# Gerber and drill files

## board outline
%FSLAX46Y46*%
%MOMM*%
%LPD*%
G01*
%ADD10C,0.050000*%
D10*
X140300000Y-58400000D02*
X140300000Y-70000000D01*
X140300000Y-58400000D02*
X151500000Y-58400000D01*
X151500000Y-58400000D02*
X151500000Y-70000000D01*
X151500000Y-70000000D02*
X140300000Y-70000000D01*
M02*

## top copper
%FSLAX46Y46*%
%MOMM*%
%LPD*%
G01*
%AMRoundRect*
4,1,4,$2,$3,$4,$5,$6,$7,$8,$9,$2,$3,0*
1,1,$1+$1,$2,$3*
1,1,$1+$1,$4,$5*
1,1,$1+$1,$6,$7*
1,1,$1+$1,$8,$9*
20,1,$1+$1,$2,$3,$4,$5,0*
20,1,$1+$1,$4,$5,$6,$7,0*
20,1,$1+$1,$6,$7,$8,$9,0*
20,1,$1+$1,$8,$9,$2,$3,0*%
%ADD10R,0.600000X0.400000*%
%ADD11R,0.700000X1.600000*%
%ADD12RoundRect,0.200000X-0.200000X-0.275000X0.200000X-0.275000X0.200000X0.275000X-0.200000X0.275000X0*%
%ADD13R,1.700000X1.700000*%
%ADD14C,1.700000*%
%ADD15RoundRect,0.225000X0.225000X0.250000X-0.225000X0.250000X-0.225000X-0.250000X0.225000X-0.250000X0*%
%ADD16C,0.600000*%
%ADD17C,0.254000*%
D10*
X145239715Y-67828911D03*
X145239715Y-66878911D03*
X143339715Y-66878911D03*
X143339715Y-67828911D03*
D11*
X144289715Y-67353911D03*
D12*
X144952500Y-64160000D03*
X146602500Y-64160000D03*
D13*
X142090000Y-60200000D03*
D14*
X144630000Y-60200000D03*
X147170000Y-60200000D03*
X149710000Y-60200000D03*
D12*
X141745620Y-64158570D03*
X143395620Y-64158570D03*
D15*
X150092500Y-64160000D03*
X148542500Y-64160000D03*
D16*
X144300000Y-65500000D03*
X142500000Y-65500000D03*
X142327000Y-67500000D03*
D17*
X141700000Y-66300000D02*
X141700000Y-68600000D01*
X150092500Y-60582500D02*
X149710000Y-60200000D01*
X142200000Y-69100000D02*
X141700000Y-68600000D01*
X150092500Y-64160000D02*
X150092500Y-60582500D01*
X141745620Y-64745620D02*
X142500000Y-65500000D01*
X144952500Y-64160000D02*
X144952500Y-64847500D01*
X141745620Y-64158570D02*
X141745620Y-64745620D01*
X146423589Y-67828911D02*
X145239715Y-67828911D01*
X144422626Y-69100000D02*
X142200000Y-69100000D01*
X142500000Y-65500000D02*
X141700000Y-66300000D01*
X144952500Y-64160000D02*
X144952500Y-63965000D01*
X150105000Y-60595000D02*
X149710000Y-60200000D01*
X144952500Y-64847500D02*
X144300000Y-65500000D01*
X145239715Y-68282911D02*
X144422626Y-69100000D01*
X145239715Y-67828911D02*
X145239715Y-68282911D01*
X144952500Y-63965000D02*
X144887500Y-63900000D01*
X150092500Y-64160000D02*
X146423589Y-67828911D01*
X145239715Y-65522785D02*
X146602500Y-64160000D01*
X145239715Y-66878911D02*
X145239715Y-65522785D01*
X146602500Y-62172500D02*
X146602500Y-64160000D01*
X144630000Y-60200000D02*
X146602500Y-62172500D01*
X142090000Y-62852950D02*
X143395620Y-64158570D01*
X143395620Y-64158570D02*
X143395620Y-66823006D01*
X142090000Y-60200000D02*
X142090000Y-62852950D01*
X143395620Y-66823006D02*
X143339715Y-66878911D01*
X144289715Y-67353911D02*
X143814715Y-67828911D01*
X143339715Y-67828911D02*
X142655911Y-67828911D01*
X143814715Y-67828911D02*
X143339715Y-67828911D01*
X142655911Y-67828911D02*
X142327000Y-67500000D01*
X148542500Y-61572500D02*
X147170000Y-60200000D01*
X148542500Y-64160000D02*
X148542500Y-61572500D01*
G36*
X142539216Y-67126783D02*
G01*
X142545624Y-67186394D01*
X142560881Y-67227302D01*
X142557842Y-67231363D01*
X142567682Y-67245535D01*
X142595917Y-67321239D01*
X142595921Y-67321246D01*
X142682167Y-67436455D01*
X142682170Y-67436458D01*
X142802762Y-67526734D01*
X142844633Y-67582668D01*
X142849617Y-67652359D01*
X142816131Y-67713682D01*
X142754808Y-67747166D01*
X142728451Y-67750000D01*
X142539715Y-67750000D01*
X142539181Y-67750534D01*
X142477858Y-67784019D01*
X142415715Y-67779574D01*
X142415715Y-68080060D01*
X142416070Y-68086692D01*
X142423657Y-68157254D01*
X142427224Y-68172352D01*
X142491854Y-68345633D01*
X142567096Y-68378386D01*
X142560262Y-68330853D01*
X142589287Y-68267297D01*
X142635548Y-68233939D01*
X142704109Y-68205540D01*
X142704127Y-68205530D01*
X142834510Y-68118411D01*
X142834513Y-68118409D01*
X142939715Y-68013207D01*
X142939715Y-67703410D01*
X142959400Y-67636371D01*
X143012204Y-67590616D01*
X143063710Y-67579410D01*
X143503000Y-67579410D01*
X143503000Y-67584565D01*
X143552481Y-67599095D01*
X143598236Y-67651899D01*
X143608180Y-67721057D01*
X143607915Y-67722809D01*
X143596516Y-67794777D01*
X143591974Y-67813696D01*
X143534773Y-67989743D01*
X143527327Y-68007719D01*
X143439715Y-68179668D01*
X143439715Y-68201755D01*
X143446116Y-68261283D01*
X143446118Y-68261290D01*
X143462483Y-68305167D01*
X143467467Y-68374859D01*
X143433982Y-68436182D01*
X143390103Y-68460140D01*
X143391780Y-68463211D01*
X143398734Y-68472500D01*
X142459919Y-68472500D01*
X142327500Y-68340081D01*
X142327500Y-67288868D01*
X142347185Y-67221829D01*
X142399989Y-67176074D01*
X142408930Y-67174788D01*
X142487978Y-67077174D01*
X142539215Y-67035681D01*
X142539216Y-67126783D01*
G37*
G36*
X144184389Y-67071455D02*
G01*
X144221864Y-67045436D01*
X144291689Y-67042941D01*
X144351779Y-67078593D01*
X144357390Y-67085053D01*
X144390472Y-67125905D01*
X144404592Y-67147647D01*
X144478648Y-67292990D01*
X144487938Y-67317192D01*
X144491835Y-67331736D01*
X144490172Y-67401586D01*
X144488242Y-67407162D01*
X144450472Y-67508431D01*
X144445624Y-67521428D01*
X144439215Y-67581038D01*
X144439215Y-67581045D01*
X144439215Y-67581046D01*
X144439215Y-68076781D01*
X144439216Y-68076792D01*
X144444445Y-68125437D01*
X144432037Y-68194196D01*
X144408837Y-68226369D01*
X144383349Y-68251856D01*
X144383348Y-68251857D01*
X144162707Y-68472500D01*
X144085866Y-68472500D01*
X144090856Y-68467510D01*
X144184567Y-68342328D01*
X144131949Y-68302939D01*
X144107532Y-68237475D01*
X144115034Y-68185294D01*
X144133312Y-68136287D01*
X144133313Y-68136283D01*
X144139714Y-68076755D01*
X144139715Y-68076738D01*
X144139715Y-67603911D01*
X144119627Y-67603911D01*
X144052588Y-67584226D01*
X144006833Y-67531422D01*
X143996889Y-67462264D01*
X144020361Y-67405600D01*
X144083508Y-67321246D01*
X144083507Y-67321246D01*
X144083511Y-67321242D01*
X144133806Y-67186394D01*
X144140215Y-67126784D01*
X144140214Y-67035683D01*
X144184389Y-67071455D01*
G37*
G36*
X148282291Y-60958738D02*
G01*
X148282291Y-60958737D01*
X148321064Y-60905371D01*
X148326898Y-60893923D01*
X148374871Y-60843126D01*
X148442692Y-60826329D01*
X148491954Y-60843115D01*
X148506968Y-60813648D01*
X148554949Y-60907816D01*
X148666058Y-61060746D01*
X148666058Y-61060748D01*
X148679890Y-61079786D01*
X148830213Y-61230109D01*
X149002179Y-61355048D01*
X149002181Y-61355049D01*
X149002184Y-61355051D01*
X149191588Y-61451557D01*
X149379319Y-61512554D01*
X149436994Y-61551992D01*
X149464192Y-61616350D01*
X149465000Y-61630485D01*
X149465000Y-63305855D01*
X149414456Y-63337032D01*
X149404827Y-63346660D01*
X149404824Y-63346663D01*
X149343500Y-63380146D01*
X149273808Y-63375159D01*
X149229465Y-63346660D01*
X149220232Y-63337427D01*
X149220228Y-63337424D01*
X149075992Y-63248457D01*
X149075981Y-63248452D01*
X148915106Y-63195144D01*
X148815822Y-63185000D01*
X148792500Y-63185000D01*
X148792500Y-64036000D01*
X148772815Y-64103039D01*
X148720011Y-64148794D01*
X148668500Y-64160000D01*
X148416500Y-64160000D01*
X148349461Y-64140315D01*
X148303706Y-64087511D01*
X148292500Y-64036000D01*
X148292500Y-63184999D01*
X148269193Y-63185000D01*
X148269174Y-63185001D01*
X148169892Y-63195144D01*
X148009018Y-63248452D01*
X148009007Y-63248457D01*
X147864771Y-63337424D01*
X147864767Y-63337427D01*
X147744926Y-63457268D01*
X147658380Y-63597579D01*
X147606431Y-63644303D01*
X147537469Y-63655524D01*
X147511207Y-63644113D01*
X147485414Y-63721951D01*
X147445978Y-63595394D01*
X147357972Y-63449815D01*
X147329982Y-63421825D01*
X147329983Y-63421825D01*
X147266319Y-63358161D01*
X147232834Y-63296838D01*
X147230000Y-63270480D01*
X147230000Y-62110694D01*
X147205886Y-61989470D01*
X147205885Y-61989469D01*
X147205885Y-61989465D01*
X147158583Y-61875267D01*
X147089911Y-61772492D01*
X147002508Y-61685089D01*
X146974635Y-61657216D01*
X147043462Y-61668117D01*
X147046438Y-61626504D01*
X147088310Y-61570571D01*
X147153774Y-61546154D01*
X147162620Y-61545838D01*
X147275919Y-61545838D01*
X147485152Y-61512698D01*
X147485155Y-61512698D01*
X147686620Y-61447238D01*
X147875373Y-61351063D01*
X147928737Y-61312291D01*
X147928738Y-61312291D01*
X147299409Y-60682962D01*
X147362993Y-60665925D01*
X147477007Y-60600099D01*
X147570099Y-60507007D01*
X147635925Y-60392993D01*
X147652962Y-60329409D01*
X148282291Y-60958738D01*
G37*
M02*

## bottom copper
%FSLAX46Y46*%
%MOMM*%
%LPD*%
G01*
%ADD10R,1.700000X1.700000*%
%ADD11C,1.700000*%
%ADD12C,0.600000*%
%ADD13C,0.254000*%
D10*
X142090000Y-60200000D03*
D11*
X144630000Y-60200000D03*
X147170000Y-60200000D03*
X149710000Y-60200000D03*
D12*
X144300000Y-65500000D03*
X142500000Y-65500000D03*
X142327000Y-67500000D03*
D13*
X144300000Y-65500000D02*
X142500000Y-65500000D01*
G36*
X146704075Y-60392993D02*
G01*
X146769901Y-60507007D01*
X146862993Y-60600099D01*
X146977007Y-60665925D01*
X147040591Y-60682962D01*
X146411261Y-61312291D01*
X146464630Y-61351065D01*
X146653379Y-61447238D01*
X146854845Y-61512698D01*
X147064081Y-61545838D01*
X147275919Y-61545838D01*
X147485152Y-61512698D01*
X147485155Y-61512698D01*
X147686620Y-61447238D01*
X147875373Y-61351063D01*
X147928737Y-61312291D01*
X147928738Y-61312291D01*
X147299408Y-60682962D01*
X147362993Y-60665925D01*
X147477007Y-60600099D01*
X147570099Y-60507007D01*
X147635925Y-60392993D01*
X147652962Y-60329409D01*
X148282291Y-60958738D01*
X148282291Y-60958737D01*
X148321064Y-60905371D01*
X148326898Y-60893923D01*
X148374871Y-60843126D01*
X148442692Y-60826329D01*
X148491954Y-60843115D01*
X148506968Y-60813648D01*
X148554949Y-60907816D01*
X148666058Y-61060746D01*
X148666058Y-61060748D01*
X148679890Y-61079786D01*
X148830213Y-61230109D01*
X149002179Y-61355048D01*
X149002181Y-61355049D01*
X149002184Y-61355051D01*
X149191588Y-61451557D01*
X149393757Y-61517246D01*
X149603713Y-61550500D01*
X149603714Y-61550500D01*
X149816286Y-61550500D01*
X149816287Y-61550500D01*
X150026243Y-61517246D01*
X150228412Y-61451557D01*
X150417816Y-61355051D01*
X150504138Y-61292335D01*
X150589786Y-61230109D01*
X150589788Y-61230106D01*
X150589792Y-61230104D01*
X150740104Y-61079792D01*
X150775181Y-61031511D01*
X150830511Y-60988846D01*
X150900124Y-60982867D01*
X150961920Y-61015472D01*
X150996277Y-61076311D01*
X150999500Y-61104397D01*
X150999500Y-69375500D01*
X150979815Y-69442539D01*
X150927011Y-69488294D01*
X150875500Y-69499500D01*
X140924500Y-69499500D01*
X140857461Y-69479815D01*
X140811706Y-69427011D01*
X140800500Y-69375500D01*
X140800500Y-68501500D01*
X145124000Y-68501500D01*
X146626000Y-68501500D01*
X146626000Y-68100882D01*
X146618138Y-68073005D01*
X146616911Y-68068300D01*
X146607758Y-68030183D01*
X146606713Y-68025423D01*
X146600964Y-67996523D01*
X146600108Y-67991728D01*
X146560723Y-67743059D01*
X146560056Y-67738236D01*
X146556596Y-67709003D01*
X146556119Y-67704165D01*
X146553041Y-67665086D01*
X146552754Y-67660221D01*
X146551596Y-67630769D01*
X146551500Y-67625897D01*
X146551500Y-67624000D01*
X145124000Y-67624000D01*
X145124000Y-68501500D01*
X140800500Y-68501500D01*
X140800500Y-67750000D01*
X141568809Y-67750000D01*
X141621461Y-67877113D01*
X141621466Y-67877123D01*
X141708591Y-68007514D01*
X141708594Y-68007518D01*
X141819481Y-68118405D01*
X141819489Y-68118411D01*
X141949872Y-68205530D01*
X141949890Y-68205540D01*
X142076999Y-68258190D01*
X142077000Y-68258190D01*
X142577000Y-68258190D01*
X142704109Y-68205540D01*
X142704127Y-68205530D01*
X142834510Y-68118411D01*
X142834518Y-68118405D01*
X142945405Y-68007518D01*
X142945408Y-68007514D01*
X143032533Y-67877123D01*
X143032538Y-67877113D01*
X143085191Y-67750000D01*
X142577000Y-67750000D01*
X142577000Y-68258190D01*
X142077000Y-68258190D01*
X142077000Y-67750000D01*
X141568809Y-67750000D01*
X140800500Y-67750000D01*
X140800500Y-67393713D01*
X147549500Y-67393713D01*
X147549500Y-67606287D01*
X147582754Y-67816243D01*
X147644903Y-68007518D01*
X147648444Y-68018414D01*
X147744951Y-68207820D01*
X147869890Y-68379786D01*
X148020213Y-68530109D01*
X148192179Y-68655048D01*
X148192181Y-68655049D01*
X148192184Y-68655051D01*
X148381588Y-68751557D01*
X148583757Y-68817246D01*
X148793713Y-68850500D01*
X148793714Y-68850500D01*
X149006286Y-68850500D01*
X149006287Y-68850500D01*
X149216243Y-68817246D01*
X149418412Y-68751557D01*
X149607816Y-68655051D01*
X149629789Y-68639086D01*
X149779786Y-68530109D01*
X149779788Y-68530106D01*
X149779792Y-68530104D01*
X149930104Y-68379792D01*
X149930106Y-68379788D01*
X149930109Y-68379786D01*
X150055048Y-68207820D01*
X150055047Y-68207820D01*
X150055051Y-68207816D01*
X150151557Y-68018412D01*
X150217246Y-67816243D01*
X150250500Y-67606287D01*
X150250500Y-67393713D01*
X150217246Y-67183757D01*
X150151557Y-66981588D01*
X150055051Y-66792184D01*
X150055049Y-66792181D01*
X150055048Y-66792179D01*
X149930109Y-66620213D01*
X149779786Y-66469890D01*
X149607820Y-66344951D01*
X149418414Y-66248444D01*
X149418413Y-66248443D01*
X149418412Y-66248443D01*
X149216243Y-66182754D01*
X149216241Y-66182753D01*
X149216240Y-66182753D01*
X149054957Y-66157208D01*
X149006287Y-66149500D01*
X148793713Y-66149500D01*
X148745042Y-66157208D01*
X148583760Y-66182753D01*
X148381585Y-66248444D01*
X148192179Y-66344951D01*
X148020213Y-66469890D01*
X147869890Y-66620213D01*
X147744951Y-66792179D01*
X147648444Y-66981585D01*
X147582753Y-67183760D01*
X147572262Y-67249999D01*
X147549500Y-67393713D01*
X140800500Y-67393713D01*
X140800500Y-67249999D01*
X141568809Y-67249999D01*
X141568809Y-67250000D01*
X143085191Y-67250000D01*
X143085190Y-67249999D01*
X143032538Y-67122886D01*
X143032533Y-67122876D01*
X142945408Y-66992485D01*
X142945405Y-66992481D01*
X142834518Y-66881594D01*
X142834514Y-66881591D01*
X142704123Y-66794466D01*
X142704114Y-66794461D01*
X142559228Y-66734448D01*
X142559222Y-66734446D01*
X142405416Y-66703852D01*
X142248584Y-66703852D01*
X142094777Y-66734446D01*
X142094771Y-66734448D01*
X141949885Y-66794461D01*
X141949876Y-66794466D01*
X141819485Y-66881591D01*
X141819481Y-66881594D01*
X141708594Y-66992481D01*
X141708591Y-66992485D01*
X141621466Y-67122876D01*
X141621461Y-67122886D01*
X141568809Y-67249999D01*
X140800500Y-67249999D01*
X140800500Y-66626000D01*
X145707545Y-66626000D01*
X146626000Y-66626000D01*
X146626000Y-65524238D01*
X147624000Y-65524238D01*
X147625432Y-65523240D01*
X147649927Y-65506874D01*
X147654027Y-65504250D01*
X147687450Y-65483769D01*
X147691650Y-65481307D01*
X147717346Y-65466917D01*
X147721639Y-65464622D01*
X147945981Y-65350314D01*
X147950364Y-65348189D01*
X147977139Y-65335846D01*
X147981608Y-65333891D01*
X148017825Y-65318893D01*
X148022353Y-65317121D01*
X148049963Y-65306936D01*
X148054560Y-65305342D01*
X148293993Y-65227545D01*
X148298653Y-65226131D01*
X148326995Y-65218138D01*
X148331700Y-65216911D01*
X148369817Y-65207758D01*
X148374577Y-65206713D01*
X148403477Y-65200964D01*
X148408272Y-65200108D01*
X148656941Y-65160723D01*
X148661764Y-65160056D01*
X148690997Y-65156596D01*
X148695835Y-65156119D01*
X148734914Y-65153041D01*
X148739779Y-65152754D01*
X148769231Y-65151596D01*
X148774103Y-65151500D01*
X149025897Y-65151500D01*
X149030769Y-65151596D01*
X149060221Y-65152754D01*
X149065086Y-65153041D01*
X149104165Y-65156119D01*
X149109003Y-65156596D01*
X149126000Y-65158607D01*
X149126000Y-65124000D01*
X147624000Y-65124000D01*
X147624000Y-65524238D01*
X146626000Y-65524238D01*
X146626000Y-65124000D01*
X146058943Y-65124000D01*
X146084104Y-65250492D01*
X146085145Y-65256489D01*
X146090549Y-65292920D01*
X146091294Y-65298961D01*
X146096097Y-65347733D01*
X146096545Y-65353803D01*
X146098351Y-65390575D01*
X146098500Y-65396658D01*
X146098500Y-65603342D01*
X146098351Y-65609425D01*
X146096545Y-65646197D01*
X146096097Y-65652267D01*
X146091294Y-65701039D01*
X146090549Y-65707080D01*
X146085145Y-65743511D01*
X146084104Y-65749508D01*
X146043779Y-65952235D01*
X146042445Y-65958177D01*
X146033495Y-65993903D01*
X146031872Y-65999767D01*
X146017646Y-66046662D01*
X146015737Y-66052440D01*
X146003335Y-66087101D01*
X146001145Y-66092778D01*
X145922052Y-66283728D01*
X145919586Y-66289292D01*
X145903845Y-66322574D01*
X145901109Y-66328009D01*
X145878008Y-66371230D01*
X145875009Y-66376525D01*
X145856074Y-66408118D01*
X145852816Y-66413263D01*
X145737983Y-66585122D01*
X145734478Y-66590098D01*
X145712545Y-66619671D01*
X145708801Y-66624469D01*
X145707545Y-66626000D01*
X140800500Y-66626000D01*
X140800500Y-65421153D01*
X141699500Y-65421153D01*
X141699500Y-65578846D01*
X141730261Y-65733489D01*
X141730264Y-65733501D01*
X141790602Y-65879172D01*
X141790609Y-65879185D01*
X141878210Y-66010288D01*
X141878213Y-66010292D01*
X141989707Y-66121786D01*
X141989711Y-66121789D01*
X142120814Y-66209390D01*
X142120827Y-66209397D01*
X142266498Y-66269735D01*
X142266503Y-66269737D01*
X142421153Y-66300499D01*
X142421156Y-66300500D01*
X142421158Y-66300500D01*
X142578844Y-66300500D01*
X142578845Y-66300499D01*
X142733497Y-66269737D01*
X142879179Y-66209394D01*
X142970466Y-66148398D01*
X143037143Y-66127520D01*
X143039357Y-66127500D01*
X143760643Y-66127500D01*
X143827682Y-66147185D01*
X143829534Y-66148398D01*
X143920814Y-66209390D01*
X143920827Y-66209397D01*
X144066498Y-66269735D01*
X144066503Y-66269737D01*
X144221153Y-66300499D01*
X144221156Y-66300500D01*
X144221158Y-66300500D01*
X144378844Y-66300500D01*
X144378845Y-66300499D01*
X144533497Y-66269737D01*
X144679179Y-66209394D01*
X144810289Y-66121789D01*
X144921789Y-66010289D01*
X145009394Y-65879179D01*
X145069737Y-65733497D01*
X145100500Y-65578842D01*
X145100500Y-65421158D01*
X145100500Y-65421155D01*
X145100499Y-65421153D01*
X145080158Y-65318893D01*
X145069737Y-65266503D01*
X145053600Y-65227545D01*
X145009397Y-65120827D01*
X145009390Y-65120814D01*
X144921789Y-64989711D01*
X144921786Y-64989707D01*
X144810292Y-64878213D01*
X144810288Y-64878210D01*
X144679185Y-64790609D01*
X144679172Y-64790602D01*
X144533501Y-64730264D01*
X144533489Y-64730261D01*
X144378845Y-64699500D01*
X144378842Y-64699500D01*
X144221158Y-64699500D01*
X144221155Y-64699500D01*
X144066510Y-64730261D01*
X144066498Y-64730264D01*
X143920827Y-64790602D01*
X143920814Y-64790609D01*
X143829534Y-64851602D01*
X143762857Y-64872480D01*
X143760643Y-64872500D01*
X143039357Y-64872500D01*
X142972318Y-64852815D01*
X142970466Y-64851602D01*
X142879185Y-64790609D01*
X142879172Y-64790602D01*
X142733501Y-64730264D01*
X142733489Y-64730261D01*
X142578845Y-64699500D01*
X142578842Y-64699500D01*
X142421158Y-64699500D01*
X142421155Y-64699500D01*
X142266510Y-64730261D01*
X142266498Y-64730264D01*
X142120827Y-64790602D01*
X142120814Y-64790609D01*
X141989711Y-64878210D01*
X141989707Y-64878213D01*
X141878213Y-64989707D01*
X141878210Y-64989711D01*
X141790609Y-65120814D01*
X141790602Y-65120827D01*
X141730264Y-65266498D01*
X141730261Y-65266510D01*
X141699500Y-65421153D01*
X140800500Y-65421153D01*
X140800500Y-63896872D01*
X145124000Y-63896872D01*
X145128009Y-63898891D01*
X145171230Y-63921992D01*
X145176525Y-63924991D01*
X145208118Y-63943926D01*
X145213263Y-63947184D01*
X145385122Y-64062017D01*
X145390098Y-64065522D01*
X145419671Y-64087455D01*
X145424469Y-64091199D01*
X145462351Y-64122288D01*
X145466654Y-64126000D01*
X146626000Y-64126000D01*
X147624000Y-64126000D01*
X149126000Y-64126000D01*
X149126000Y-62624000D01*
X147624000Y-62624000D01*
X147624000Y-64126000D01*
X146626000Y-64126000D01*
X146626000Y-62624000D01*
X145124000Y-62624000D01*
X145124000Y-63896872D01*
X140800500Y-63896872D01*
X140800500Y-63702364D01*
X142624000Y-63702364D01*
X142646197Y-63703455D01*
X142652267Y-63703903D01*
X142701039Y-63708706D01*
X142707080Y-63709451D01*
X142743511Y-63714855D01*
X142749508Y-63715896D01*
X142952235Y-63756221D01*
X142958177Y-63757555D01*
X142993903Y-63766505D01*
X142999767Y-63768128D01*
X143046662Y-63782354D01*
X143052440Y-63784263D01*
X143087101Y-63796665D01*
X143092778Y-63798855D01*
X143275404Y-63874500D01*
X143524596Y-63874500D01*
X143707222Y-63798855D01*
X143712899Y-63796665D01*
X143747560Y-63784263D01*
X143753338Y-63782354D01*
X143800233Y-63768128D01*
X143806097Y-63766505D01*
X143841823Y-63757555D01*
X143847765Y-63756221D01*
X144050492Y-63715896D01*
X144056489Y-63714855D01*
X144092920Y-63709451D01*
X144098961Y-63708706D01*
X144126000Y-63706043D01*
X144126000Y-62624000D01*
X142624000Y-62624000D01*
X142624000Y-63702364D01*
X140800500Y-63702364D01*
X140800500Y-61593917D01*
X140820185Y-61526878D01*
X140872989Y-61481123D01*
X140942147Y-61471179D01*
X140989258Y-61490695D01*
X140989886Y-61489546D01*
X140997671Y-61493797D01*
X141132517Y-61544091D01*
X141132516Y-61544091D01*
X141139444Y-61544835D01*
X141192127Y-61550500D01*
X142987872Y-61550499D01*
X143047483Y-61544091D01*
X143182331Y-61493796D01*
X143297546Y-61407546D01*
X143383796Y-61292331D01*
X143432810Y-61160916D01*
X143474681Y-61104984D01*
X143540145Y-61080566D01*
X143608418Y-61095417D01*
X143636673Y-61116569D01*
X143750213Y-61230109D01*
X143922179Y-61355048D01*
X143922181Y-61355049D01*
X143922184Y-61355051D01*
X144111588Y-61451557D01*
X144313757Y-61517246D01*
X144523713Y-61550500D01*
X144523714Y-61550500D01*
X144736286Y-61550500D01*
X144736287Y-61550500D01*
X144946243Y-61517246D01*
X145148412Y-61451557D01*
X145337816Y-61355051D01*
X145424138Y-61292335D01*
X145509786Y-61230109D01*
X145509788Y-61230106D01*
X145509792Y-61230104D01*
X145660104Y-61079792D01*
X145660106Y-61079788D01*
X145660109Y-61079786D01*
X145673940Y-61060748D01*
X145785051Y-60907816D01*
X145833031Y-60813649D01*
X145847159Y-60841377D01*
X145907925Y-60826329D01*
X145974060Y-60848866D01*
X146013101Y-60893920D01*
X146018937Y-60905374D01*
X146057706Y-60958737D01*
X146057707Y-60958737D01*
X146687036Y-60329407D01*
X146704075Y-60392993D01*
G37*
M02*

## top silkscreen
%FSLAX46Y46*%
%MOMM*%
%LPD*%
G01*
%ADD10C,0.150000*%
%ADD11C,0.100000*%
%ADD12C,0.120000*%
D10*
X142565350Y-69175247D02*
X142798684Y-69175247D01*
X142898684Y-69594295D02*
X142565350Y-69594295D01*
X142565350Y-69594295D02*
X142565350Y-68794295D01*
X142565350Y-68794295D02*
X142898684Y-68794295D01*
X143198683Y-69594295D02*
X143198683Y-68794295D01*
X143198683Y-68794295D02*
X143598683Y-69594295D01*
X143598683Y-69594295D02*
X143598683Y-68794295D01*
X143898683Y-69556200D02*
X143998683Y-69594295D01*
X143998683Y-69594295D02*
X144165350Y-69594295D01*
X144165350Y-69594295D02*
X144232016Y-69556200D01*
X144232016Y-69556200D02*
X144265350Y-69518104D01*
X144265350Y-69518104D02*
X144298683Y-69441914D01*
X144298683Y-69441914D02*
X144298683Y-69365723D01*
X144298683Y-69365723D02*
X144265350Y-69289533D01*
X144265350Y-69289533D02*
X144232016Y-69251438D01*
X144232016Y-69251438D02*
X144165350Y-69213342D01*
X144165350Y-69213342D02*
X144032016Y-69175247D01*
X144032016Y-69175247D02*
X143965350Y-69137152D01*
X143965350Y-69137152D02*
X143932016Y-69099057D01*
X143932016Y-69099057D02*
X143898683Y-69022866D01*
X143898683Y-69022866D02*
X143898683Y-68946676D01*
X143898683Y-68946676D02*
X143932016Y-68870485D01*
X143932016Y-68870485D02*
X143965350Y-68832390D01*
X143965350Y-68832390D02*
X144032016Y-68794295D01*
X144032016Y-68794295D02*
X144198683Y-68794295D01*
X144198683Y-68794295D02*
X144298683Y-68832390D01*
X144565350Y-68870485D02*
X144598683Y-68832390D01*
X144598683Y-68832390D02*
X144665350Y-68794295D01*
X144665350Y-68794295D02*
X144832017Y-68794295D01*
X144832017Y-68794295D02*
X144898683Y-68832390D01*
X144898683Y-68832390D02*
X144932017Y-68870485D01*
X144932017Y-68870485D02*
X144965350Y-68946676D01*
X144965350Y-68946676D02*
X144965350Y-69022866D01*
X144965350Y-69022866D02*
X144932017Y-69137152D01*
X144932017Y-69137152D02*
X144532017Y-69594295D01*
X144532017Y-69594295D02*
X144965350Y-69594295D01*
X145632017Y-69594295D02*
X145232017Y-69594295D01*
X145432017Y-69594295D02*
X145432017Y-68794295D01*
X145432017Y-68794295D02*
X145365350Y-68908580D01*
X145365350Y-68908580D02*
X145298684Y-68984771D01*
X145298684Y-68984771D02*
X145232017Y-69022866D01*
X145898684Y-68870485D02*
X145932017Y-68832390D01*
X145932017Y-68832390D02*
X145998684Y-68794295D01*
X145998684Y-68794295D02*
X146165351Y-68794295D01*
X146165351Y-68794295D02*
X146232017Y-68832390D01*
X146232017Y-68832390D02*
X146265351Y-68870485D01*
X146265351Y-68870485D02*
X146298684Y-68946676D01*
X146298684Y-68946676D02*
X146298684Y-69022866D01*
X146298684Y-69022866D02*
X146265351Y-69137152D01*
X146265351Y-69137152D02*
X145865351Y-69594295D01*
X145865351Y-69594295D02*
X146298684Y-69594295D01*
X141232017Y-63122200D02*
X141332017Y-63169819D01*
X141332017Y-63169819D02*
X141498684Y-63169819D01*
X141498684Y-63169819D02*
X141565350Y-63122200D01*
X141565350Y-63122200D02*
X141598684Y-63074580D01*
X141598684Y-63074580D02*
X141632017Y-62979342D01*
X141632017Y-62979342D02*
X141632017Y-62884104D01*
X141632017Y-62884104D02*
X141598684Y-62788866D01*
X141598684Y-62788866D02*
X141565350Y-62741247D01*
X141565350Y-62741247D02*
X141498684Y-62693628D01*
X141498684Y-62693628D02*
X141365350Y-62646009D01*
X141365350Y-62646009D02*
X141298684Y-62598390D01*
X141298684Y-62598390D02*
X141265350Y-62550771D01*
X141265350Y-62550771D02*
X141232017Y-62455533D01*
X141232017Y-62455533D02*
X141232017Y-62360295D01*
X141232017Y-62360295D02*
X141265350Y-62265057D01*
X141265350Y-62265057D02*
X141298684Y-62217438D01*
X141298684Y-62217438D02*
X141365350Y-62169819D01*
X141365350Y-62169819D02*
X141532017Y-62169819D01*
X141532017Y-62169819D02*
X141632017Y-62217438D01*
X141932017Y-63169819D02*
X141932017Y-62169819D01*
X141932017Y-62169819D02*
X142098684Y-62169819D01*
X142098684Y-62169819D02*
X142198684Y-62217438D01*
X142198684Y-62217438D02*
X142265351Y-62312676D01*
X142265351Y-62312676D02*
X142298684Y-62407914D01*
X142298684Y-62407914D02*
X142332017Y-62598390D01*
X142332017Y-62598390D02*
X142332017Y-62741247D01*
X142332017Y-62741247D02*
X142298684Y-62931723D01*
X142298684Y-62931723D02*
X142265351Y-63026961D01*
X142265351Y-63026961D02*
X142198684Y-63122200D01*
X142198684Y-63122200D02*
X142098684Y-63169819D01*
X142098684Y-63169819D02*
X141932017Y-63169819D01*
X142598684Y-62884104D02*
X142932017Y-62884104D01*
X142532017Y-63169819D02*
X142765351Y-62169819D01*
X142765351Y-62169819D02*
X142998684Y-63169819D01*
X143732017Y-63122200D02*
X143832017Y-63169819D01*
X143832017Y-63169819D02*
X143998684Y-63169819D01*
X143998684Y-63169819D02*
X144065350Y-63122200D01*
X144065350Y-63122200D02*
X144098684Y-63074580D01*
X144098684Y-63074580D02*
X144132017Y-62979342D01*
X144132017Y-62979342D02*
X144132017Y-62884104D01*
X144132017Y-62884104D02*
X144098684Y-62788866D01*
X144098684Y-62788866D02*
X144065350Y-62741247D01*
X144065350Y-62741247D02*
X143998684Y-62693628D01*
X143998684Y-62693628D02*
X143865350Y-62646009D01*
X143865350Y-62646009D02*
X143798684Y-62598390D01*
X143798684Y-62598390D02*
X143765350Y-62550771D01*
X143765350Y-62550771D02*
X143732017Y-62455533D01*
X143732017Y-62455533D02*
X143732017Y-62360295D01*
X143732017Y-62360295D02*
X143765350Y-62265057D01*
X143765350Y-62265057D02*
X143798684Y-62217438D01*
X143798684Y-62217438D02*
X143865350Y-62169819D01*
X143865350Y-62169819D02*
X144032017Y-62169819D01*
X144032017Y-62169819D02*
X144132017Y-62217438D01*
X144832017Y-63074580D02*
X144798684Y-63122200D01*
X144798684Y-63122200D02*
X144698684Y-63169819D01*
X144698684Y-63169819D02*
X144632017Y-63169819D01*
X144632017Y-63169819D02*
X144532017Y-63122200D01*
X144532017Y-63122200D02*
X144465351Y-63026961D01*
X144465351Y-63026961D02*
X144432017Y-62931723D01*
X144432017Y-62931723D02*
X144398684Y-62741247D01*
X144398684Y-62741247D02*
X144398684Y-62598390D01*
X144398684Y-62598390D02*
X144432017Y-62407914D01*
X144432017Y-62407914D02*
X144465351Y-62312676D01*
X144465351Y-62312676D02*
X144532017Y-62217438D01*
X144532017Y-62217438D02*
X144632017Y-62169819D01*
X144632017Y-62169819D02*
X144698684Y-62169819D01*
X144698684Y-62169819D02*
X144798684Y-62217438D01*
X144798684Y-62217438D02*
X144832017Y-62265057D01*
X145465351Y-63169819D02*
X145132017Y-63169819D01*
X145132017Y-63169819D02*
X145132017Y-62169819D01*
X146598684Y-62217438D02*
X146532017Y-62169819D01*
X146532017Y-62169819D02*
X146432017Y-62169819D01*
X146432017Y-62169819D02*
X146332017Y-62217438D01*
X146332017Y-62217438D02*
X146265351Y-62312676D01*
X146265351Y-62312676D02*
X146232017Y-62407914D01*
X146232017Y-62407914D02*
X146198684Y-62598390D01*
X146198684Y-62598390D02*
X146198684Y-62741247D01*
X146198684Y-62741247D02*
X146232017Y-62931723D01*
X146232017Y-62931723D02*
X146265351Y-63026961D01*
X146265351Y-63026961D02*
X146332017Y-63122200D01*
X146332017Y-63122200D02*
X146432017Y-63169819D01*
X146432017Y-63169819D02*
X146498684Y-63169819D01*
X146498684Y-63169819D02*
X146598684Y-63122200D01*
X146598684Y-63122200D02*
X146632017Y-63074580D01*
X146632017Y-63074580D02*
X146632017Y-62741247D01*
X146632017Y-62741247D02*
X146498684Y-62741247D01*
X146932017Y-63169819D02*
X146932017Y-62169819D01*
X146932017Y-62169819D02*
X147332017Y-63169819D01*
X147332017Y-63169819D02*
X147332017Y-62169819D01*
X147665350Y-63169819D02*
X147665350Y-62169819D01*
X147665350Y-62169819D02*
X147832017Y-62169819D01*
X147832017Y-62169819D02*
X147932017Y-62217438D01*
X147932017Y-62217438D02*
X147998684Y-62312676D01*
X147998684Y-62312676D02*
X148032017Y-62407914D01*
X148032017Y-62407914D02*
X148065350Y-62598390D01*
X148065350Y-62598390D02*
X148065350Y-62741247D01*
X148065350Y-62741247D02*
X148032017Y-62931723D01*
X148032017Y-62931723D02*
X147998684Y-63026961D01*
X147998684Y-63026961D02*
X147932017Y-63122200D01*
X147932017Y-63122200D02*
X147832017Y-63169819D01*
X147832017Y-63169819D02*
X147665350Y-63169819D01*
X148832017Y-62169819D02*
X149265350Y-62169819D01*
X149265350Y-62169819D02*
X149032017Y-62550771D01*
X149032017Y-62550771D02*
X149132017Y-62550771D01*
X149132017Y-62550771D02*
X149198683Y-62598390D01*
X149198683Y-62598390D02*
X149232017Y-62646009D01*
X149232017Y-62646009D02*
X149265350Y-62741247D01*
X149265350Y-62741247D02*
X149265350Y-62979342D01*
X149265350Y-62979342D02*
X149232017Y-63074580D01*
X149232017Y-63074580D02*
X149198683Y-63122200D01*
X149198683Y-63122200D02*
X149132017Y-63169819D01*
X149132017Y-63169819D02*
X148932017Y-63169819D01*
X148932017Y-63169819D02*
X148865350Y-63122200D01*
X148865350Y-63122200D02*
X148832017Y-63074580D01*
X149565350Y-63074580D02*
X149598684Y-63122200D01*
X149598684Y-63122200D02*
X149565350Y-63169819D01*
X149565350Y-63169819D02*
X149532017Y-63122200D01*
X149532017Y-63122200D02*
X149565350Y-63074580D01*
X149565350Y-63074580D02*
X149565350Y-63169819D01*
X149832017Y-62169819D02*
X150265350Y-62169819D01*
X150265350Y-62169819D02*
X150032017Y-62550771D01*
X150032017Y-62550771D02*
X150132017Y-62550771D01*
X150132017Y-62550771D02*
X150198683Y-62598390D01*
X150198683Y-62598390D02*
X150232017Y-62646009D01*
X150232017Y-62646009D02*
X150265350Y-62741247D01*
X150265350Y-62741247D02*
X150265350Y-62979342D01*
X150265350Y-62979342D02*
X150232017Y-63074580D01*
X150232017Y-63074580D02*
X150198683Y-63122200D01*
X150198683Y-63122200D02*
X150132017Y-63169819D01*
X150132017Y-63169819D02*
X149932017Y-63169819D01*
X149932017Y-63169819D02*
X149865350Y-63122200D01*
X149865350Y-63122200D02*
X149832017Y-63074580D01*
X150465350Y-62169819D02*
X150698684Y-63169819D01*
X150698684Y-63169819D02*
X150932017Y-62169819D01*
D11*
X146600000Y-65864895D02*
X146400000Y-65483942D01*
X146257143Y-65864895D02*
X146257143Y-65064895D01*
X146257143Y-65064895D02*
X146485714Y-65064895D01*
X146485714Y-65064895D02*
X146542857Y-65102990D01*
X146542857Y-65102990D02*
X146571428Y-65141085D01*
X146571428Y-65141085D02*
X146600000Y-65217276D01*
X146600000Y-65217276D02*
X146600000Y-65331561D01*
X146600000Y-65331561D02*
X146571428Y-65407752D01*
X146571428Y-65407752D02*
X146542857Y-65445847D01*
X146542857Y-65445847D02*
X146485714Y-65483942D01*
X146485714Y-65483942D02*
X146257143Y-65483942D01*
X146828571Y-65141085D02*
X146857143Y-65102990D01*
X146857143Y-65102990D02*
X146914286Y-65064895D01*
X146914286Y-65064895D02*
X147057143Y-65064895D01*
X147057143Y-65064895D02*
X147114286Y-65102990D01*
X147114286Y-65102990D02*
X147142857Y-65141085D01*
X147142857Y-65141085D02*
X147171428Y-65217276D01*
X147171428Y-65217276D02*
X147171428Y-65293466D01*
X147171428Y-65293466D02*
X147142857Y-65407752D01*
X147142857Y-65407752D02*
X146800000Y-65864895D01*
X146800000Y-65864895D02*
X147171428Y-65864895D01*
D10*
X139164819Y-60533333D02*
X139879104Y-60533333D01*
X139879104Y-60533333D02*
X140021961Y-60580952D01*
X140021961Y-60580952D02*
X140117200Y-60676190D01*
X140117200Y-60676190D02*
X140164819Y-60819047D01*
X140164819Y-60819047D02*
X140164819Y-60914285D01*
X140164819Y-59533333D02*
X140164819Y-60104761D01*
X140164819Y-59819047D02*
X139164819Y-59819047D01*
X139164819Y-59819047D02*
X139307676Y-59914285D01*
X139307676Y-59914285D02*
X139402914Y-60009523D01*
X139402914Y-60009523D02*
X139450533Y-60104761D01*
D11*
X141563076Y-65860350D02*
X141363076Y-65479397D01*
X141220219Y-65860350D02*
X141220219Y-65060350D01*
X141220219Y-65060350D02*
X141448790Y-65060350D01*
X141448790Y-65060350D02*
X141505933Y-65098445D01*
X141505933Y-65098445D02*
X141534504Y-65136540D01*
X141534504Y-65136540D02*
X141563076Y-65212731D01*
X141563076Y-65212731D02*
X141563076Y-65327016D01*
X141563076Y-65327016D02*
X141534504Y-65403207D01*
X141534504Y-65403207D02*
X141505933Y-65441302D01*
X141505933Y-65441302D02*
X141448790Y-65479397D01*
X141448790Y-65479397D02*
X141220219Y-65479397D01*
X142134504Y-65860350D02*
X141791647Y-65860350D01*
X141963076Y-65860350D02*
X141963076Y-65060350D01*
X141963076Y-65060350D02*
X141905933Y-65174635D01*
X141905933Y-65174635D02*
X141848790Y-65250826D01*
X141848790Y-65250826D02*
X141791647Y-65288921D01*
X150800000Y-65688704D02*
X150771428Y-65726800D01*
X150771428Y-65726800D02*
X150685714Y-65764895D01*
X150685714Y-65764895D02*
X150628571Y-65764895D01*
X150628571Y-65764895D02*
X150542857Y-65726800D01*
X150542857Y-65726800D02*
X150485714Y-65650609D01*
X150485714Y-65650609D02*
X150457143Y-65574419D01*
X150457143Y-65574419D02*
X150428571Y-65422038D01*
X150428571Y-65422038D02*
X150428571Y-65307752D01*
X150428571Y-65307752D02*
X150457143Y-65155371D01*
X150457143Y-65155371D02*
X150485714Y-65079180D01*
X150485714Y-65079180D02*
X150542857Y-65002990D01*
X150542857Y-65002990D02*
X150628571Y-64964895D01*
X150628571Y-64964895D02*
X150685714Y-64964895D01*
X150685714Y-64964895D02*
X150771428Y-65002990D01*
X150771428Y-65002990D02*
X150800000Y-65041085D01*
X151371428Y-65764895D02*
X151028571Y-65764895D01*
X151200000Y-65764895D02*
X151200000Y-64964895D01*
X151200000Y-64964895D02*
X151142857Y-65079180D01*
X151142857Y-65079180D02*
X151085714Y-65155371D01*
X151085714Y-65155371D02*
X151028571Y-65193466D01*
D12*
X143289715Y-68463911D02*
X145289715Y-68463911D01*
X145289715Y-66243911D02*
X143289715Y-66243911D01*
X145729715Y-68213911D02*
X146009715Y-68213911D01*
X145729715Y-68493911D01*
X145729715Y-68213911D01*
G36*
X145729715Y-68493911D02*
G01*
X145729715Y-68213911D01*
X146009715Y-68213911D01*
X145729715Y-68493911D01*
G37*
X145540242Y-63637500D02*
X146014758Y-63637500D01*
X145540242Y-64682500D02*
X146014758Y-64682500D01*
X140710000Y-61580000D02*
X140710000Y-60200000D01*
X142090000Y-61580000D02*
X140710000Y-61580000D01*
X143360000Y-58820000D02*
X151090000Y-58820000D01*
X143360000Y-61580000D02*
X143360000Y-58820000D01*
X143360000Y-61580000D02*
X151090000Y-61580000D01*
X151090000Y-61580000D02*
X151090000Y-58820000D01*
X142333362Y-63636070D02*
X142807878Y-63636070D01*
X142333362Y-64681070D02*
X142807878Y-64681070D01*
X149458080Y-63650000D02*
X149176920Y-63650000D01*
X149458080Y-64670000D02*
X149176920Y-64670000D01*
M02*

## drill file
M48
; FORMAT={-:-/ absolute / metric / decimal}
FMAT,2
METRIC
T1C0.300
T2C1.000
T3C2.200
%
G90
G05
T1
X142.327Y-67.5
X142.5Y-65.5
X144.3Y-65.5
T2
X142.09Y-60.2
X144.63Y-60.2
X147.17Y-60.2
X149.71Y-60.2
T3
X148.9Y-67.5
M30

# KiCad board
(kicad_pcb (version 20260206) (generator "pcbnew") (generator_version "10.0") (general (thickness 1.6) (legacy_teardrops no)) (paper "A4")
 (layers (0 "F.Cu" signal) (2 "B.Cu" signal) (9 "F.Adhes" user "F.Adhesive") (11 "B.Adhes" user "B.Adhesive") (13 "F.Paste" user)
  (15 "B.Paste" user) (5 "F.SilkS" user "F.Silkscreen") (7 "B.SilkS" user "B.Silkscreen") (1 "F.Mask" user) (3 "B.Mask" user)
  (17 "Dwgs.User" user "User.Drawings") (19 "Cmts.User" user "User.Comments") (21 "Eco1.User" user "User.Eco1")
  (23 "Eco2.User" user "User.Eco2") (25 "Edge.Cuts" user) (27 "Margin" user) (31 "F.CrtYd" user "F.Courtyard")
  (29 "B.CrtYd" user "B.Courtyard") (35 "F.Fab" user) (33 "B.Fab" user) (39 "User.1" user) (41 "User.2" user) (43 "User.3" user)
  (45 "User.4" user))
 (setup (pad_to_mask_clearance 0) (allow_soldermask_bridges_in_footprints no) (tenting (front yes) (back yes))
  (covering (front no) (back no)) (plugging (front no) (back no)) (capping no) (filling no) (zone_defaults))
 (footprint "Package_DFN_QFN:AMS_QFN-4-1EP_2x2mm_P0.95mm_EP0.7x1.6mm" (layer "F.Cu") (at 144.289715 67.353911 180)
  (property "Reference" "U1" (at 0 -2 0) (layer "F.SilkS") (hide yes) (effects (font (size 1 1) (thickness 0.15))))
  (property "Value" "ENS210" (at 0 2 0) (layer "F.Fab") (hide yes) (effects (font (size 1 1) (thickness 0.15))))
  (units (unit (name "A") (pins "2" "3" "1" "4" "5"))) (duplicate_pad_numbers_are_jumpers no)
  (fp_line (start 1 -1.11) (end -1 -1.11) (stroke (width 0.12) (type solid)) (layer "F.SilkS"))
  (fp_line (start -1 1.11) (end 1 1.11) (stroke (width 0.12) (type solid)) (layer "F.SilkS"))
  (fp_poly
   (pts (xy -1.44 -0.86) (xy -1.72 -0.86) (xy -1.44 -1.14) (xy -1.44 -0.86)) (stroke (width 0.12) (type solid)) (fill yes) (layer "F.SilkS"))
  (pad "" smd rect (at 0 0 180) (size 0.35 0.8) (layers "F.Paste"))
  (pad "1" smd rect (at -0.95 -0.475 180) (size 0.6 0.4) (layers "F.Cu" "F.Mask" "F.Paste") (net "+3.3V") (solder_paste_margin -0.05))
  (pad "2" smd rect (at -0.95 0.475 180) (size 0.6 0.4) (layers "F.Cu" "F.Mask" "F.Paste") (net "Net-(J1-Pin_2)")
   (solder_paste_margin -0.05))
  (pad "3" smd rect (at 0.95 0.475 180) (size 0.6 0.4) (layers "F.Cu" "F.Mask" "F.Paste") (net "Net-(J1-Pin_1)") (solder_paste_margin -0.05))
  (pad "4" smd rect (at 0.95 -0.475 180) (size 0.6 0.4) (layers "F.Cu" "F.Mask" "F.Paste") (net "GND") (solder_paste_margin -0.05))
  (pad "5" smd rect (at 0 0 180) (size 0.7 1.6) (layers "F.Cu" "F.Mask") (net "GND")))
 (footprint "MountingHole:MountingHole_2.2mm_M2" (layer "F.Cu") (at 148.9 67.5)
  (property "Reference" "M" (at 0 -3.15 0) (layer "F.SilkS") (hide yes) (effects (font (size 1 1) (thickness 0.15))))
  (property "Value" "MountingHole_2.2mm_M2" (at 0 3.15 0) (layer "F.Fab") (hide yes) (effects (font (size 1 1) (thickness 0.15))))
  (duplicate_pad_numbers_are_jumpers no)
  (pad "" np_thru_hole circle (at 0 0) (size 2.2 2.2) (drill 2.2) (layers "*.Cu" "*.Mask")))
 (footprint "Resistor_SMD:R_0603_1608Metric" (layer "F.Cu") (at 145.7775 64.16)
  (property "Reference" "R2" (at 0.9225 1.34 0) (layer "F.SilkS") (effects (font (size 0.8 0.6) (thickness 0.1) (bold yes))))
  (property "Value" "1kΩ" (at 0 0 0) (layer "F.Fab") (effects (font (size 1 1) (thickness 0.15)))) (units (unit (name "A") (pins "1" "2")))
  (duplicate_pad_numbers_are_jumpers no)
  (fp_line (start -0.237258 -0.5225) (end 0.237258 -0.5225) (stroke (width 0.12) (type solid)) (layer "F.SilkS"))
  (fp_line (start -0.237258 0.5225) (end 0.237258 0.5225) (stroke (width 0.12) (type solid)) (layer "F.SilkS"))
  (pad "1" smd roundrect (at -0.825 0) (size 0.8 0.95) (layers "F.Cu" "F.Mask" "F.Paste") (roundrect_rratio 0.25) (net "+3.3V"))
  (pad "2" smd roundrect (at 0.825 0) (size 0.8 0.95) (layers "F.Cu" "F.Mask" "F.Paste") (roundrect_rratio 0.25) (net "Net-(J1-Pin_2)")))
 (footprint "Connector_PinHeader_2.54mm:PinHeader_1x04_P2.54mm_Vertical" (layer "F.Cu") (at 142.09 60.2 90)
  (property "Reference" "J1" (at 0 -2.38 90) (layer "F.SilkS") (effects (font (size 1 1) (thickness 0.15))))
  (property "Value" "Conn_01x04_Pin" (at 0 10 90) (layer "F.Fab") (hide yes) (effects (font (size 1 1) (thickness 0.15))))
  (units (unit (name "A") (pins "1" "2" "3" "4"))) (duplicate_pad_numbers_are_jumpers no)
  (fp_line (start -1.38 -1.38) (end 0 -1.38) (stroke (width 0.12) (type solid)) (layer "F.SilkS"))
  (fp_line (start -1.38 0) (end -1.38 -1.38) (stroke (width 0.12) (type solid)) (layer "F.SilkS"))
  (fp_line (start 1.38 1.27) (end 1.38 9) (stroke (width 0.12) (type solid)) (layer "F.SilkS"))
  (fp_line (start -1.38 1.27) (end 1.38 1.27) (stroke (width 0.12) (type solid)) (layer "F.SilkS"))
  (fp_line (start -1.38 1.27) (end -1.38 9) (stroke (width 0.12) (type solid)) (layer "F.SilkS"))
  (fp_line (start -1.38 9) (end 1.38 9) (stroke (width 0.12) (type solid)) (layer "F.SilkS"))
  (pad "1" thru_hole rect (at 0 0 90) (size 1.7 1.7) (drill 1) (layers "*.Cu" "*.Mask") (remove_unused_layers no) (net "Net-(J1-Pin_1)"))
  (pad "2" thru_hole circle (at 0 2.54 90) (size 1.7 1.7) (drill 1) (layers "*.Cu" "*.Mask") (remove_unused_layers no)
   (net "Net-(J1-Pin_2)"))
  (pad "3" thru_hole circle (at 0 5.08 90) (size 1.7 1.7) (drill 1) (layers "*.Cu" "*.Mask") (remove_unused_layers no) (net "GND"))
  (pad "4" thru_hole circle (at 0 7.62 90) (size 1.7 1.7) (drill 1) (layers "*.Cu" "*.Mask") (remove_unused_layers no) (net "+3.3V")))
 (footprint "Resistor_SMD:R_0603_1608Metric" (layer "F.Cu") (at 142.57062 64.15857)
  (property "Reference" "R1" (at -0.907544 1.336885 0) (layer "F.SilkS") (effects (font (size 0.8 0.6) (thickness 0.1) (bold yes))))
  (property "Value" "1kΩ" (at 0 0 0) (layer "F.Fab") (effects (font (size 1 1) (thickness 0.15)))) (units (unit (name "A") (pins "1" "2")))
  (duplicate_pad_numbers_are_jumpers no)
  (fp_line (start -0.237258 -0.5225) (end 0.237258 -0.5225) (stroke (width 0.12) (type solid)) (layer "F.SilkS"))
  (fp_line (start -0.237258 0.5225) (end 0.237258 0.5225) (stroke (width 0.12) (type solid)) (layer "F.SilkS"))
  (pad "1" smd roundrect (at -0.825 0) (size 0.8 0.95) (layers "F.Cu" "F.Mask" "F.Paste") (roundrect_rratio 0.25) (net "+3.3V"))
  (pad "2" smd roundrect (at 0.825 0) (size 0.8 0.95) (layers "F.Cu" "F.Mask" "F.Paste") (roundrect_rratio 0.25) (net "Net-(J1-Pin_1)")))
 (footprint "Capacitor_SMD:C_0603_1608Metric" (layer "F.Cu") (at 149.3175 64.16 180)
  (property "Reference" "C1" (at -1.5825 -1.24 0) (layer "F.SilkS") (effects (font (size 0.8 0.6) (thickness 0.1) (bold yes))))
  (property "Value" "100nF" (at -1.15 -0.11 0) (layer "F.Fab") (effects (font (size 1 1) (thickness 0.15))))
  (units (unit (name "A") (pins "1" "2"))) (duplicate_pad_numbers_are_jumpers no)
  (fp_line (start -0.14058 0.51) (end 0.14058 0.51) (stroke (width 0.12) (type solid)) (layer "F.SilkS"))
  (fp_line (start -0.14058 -0.51) (end 0.14058 -0.51) (stroke (width 0.12) (type solid)) (layer "F.SilkS"))
  (pad "1" smd roundrect (at -0.775 0 180) (size 0.9 0.95) (layers "F.Cu" "F.Mask" "F.Paste") (roundrect_rratio 0.25) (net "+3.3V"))
  (pad "2" smd roundrect (at 0.775 0 180) (size 0.9 0.95) (layers "F.Cu" "F.Mask" "F.Paste") (roundrect_rratio 0.25) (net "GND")))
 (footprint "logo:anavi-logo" (layer "B.Cu") (at 142.25 64.8)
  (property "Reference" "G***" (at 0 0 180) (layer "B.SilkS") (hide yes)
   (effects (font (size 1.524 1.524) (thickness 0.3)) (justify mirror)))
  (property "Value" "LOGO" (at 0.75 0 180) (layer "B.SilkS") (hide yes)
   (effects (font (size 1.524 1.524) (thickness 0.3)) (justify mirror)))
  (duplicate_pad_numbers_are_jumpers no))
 (gr_line (start 140.3 58.4) (end 140.3 70) (stroke (width 0.05) (type default)) (layer "Edge.Cuts"))
 (gr_line (start 140.3 58.4) (end 151.5 58.4) (stroke (width 0.05) (type default)) (layer "Edge.Cuts"))
 (gr_line (start 151.5 58.4) (end 151.5 70) (stroke (width 0.05) (type default)) (layer "Edge.Cuts"))
 (gr_line (start 151.5 70) (end 140.3 70) (stroke (width 0.05) (type default)) (layer "Edge.Cuts"))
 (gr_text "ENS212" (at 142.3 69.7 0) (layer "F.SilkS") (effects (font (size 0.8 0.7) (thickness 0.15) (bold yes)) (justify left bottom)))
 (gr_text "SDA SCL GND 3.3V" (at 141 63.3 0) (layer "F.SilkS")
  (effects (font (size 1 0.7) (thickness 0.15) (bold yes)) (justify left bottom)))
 (segment (start 141.7 66.3) (end 141.7 68.6) (width 0.254) (layer "F.Cu") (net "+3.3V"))
 (segment (start 150.0925 60.5825) (end 149.71 60.2) (width 0.254) (layer "F.Cu") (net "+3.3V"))
 (segment (start 142.2 69.1) (end 141.7 68.6) (width 0.254) (layer "F.Cu") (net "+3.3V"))
 (segment (start 150.0925 64.16) (end 150.0925 60.5825) (width 0.254) (layer "F.Cu") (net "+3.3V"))
 (segment (start 141.74562 64.74562) (end 142.5 65.5) (width 0.254) (layer "F.Cu") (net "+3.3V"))
 (segment (start 144.9525 64.16) (end 144.9525 64.8475) (width 0.254) (layer "F.Cu") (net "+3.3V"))
 (segment (start 141.74562 64.15857) (end 141.74562 64.74562) (width 0.254) (layer "F.Cu") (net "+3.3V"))
 (segment (start 146.423589 67.828911) (end 145.239715 67.828911) (width 0.254) (layer "F.Cu") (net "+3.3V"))
 (segment (start 144.422626 69.1) (end 142.2 69.1) (width 0.254) (layer "F.Cu") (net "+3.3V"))
 (segment (start 142.5 65.5) (end 141.7 66.3) (width 0.254) (layer "F.Cu") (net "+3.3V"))
 (segment (start 144.9525 64.16) (end 144.9525 63.965) (width 0.254) (layer "F.Cu") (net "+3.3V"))
 (segment (start 150.105 60.595) (end 149.71 60.2) (width 0.254) (layer "F.Cu") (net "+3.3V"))
 (segment (start 144.9525 64.8475) (end 144.3 65.5) (width 0.254) (layer "F.Cu") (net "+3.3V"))
 (segment (start 145.239715 68.282911) (end 144.422626 69.1) (width 0.254) (layer "F.Cu") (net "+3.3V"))
 (segment (start 145.239715 67.828911) (end 145.239715 68.282911) (width 0.254) (layer "F.Cu") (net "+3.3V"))
 (segment (start 144.9525 63.965) (end 144.8875 63.9) (width 0.254) (layer "F.Cu") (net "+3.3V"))
 (segment (start 150.0925 64.16) (end 146.423589 67.828911) (width 0.254) (layer "F.Cu") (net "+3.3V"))
 (via (at 144.3 65.5) (size 0.6) (drill 0.3) (layers "F.Cu" "B.Cu") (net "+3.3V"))
 (via (at 142.5 65.5) (size 0.6) (drill 0.3) (layers "F.Cu" "B.Cu") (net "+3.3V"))
 (segment (start 144.3 65.5) (end 142.5 65.5) (width 0.254) (layer "B.Cu") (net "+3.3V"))
 (segment (start 145.239715 65.522785) (end 146.6025 64.16) (width 0.254) (layer "F.Cu") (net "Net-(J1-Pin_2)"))
 (segment (start 145.239715 66.878911) (end 145.239715 65.522785) (width 0.254) (layer "F.Cu") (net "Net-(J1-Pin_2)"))
 (segment (start 146.6025 62.1725) (end 146.6025 64.16) (width 0.254) (layer "F.Cu") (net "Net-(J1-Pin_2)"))
 (segment (start 144.63 60.2) (end 146.6025 62.1725) (width 0.254) (layer "F.Cu") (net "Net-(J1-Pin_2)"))
 (segment (start 142.09 62.85295) (end 143.39562 64.15857) (width 0.254) (layer "F.Cu") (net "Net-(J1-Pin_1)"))
 (segment (start 143.39562 64.15857) (end 143.39562 66.823006) (width 0.254) (layer "F.Cu") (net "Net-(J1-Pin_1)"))
 (segment (start 142.09 60.2) (end 142.09 62.85295) (width 0.254) (layer "F.Cu") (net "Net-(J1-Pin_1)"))
 (segment (start 143.39562 66.823006) (end 143.339715 66.878911) (width 0.254) (layer "F.Cu") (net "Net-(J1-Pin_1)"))
 (segment (start 144.289715 67.353911) (end 143.814715 67.828911) (width 0.254) (layer "F.Cu") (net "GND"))
 (segment (start 143.339715 67.828911) (end 142.655911 67.828911) (width 0.254) (layer "F.Cu") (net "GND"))
 (segment (start 143.814715 67.828911) (end 143.339715 67.828911) (width 0.254) (layer "F.Cu") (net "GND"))
 (segment (start 142.655911 67.828911) (end 142.327 67.5) (width 0.254) (layer "F.Cu") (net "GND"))
 (segment (start 148.5425 61.5725) (end 147.17 60.2) (width 0.254) (layer "F.Cu") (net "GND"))
 (segment (start 148.5425 64.16) (end 148.5425 61.5725) (width 0.254) (layer "F.Cu") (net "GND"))
 (via (at 142.327 67.5) (size 0.6) (drill 0.3) (layers "F.Cu" "B.Cu") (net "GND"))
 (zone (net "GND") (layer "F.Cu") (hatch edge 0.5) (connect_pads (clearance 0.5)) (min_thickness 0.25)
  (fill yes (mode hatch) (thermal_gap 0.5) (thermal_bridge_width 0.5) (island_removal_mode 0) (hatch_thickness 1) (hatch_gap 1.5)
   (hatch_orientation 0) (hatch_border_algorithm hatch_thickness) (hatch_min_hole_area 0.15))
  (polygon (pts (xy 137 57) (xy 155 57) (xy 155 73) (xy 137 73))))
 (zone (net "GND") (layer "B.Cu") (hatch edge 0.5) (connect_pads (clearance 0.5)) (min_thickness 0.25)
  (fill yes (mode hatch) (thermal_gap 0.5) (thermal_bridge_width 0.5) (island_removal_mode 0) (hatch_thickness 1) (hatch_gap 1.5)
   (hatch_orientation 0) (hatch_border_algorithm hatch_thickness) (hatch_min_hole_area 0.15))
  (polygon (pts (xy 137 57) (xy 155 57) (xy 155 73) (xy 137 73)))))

